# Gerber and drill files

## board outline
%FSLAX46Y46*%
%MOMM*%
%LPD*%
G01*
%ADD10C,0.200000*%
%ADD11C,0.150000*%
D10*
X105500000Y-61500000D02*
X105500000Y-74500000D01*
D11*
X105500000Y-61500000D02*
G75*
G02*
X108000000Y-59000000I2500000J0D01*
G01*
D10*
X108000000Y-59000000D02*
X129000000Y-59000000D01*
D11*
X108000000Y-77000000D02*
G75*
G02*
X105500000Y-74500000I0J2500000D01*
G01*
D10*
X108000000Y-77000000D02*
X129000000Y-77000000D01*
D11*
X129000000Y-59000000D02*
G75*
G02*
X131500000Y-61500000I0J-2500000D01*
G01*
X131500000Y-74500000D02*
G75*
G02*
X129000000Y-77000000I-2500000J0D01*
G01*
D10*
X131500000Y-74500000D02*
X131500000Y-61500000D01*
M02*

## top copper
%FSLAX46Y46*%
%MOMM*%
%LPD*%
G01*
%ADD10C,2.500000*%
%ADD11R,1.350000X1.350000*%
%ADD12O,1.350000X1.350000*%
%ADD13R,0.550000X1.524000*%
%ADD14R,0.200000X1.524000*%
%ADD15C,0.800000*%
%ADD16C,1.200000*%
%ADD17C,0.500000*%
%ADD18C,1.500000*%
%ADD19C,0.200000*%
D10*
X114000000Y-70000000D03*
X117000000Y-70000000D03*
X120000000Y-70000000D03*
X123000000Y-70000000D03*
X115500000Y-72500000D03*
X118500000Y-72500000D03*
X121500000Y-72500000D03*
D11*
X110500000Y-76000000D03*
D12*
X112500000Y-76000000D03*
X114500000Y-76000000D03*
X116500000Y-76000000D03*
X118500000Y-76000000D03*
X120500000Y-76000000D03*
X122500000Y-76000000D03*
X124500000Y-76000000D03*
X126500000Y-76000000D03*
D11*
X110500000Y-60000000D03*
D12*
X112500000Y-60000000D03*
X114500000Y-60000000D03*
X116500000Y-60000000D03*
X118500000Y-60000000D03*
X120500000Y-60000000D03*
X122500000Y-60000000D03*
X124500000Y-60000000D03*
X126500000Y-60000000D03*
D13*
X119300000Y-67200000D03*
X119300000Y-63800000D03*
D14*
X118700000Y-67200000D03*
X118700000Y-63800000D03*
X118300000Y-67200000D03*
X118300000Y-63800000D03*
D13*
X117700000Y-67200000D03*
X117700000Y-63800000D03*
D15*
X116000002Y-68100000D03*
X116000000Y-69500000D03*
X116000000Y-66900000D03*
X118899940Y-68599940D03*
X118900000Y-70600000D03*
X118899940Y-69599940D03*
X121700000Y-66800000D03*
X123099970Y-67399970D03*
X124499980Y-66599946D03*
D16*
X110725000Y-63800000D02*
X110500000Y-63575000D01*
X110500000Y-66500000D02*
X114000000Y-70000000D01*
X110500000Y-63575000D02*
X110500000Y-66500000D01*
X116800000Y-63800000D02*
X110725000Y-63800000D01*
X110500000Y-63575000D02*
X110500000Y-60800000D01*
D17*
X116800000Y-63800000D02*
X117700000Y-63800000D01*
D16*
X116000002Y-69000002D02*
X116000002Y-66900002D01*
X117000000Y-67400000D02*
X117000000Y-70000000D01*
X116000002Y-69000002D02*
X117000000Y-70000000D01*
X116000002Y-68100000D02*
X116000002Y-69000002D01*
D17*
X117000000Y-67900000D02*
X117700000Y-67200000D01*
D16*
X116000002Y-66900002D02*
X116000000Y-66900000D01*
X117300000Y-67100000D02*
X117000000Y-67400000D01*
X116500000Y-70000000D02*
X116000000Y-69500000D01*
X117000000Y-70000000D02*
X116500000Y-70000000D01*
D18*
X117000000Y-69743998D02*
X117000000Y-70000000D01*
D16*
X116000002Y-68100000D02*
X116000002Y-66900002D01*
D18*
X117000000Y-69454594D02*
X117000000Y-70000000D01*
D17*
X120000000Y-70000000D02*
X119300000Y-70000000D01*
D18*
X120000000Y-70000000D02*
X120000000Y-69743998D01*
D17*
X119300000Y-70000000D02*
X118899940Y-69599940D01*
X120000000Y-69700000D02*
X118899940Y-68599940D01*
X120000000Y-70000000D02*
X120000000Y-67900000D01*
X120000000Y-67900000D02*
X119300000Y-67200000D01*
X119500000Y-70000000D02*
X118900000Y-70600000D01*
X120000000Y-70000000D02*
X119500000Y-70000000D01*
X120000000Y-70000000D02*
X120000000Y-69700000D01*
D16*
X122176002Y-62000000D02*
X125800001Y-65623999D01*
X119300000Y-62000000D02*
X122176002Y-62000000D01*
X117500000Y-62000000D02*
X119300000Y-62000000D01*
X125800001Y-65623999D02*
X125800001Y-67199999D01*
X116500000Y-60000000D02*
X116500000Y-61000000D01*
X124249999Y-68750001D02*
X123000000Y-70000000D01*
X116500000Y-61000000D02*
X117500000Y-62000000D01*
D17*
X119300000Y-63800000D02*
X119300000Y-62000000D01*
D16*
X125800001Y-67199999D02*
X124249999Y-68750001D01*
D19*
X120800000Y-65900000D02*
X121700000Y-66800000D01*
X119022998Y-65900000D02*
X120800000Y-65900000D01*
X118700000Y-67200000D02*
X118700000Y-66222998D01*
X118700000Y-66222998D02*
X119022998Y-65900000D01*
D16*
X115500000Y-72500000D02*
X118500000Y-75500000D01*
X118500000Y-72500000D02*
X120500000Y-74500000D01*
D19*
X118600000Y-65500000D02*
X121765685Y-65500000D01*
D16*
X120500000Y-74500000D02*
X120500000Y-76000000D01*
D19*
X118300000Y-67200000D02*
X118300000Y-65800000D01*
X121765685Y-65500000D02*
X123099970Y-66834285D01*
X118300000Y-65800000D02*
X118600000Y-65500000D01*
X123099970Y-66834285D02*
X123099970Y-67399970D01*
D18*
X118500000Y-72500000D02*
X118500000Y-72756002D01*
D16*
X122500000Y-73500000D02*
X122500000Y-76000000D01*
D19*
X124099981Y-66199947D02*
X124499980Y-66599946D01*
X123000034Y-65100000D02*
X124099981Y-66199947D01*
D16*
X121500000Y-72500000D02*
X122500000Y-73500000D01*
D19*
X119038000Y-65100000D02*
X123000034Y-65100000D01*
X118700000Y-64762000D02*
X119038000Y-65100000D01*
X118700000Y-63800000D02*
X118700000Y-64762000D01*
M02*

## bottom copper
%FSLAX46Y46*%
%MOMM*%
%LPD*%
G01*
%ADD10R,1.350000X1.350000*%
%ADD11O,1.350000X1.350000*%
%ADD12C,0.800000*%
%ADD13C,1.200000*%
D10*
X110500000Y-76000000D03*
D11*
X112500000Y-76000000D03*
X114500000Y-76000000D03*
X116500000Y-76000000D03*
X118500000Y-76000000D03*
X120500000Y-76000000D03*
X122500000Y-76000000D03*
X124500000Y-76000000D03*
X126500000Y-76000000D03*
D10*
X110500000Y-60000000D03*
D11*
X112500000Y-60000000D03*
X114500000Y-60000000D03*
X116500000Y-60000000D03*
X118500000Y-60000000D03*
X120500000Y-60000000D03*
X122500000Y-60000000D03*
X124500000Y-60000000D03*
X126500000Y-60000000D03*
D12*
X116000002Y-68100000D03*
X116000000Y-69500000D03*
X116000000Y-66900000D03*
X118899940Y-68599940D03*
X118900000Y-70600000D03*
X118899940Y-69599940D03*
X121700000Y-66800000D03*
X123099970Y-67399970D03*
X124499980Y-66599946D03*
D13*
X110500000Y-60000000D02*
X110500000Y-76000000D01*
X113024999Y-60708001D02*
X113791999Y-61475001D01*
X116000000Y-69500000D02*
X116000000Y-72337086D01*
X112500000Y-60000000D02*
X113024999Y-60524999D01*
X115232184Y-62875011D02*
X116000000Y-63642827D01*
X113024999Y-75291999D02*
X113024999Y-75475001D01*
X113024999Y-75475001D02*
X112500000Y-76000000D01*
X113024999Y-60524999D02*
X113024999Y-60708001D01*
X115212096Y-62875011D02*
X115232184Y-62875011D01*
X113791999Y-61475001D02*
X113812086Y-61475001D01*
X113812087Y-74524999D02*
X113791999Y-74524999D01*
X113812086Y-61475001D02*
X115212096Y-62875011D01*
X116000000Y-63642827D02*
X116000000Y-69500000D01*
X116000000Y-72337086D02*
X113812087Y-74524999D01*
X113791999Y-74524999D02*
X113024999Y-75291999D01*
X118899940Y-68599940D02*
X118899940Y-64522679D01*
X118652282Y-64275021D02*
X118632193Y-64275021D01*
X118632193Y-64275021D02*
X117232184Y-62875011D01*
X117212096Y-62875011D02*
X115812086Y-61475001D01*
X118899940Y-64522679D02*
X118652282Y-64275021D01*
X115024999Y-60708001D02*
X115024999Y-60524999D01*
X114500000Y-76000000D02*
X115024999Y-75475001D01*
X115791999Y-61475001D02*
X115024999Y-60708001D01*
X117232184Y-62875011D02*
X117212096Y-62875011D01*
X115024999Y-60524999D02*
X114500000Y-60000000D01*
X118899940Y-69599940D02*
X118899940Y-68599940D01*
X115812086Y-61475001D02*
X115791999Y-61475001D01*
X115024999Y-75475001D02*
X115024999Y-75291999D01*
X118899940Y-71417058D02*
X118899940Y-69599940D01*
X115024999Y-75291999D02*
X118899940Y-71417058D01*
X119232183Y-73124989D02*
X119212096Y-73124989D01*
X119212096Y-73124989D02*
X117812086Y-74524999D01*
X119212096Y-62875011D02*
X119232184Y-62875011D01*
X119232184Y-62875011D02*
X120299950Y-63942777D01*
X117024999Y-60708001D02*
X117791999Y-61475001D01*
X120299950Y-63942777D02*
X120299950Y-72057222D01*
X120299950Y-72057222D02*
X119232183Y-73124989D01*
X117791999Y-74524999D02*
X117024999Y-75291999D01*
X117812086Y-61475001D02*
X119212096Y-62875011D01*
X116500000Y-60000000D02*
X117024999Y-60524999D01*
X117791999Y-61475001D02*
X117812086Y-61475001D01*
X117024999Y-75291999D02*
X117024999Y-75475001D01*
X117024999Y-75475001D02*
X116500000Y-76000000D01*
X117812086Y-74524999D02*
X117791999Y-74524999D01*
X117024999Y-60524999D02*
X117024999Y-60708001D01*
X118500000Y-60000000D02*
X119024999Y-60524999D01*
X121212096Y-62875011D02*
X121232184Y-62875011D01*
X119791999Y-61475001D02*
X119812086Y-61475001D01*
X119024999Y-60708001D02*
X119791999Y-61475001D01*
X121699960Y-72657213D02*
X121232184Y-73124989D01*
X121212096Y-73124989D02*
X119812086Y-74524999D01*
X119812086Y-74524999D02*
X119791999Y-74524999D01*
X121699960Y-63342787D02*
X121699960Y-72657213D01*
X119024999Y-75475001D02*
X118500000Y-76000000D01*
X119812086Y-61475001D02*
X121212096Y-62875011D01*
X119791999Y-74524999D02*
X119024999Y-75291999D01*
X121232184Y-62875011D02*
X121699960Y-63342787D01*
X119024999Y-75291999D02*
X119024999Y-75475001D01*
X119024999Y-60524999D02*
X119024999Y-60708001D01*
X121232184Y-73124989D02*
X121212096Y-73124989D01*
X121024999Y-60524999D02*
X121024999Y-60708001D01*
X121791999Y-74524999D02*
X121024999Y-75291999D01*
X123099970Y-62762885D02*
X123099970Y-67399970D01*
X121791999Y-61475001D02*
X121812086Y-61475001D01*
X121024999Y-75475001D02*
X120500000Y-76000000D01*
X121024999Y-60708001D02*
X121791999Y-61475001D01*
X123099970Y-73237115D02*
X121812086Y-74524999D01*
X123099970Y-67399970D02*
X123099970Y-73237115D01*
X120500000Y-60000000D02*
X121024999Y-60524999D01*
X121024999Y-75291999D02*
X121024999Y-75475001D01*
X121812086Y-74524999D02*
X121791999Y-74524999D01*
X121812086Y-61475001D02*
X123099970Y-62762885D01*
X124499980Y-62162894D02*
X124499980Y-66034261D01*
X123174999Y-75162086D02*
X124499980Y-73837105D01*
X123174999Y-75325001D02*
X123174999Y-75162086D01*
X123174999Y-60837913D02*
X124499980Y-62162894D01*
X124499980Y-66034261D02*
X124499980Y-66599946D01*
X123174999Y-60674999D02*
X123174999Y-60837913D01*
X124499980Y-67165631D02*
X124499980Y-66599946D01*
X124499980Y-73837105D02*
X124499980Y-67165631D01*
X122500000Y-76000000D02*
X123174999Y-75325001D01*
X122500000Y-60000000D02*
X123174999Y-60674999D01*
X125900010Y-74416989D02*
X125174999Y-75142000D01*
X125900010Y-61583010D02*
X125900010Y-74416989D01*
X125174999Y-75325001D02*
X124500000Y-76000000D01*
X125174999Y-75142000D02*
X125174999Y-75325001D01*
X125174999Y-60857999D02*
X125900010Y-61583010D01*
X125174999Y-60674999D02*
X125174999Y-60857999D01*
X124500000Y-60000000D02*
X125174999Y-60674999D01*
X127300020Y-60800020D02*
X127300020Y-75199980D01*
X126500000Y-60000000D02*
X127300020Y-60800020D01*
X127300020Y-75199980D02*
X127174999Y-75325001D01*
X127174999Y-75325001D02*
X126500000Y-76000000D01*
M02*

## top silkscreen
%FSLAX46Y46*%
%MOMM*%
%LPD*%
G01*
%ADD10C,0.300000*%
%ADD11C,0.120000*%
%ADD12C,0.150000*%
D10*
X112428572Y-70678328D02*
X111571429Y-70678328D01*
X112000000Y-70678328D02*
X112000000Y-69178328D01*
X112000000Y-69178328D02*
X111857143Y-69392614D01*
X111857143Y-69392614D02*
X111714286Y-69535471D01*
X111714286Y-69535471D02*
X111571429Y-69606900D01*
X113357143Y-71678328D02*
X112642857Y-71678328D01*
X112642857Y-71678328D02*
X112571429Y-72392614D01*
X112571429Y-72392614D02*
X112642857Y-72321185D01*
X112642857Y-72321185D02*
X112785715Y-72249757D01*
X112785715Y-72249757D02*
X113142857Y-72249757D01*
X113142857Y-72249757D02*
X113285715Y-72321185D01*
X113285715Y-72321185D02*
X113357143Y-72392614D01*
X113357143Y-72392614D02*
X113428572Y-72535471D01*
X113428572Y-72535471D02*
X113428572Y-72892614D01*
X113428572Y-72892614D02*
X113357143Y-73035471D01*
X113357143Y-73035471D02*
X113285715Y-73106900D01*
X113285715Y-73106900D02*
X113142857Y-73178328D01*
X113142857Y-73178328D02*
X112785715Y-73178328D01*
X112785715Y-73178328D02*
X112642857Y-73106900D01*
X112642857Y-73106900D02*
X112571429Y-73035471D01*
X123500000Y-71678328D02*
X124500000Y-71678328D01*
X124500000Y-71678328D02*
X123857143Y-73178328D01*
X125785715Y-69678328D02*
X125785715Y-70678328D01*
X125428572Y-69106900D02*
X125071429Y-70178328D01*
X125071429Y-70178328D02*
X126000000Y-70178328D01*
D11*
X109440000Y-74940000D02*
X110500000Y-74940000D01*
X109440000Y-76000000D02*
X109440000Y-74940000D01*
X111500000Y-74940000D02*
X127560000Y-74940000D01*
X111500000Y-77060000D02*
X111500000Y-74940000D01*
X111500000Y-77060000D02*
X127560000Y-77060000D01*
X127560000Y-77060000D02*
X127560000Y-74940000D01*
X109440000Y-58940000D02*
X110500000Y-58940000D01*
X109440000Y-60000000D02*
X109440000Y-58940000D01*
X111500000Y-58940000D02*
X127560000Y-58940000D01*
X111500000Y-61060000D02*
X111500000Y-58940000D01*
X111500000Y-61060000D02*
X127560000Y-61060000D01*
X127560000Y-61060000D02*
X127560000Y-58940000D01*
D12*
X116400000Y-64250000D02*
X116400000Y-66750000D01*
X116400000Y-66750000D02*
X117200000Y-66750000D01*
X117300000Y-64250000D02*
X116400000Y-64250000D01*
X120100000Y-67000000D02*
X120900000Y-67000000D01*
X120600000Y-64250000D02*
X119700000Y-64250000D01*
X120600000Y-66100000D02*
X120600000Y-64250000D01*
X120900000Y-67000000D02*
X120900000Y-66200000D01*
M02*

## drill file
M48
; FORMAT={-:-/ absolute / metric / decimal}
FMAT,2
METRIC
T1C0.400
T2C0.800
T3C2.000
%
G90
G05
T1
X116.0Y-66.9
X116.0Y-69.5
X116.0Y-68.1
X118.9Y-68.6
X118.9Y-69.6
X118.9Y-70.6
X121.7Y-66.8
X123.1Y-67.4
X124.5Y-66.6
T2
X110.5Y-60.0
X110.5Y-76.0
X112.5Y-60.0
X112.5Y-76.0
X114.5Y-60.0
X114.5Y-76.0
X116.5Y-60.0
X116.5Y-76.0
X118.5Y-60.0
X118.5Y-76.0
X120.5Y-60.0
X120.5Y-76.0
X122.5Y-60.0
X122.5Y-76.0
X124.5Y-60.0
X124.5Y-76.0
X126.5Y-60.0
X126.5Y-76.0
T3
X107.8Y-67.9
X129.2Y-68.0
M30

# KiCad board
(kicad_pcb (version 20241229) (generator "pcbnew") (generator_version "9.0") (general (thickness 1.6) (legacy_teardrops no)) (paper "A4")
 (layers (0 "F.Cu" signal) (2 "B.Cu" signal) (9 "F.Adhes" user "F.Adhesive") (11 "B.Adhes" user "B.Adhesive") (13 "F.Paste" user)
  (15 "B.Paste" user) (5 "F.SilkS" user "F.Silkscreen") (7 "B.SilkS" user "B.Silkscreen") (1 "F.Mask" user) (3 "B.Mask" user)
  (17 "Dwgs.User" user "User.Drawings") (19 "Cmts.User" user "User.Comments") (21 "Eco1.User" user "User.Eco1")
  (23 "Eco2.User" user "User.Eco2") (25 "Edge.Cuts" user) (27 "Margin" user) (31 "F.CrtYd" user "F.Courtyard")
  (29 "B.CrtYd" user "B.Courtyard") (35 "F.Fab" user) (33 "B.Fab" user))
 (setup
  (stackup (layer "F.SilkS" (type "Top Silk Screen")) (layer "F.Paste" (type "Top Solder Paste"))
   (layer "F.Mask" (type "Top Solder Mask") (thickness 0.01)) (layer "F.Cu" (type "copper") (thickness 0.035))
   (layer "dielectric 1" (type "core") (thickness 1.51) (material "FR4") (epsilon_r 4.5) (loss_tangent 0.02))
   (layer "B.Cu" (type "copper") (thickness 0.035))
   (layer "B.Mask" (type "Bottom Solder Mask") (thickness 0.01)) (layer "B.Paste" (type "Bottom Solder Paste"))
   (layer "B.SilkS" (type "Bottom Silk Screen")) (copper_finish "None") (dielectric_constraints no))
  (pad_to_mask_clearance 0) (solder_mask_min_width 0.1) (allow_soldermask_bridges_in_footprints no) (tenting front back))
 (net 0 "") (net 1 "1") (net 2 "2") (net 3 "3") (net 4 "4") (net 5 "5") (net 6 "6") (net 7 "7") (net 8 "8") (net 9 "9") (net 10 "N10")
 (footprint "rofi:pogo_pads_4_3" (layer "F.Cu") (at 118.5 70)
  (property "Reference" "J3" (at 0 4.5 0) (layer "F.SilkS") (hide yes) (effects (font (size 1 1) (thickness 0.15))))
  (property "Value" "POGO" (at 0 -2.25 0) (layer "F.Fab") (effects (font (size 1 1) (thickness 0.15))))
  (pad "1" smd circle (at -4.5 0) (size 2.5 2.5) (layers "F.Cu" "F.Mask" "F.Paste") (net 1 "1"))
  (pad "2" smd circle (at -1.5 0) (size 2.5 2.5) (layers "F.Cu" "F.Mask" "F.Paste") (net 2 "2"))
  (pad "3" smd circle (at 1.5 0) (size 2.5 2.5) (layers "F.Cu" "F.Mask" "F.Paste") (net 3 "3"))
  (pad "4" smd circle (at 4.5 0) (size 2.5 2.5) (layers "F.Cu" "F.Mask" "F.Paste") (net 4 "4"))
  (pad "5" smd circle (at -3 2.5) (size 2.5 2.5) (layers "F.Cu" "F.Mask" "F.Paste") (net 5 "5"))
  (pad "6" smd circle (at 0 2.5) (size 2.5 2.5) (layers "F.Cu" "F.Mask" "F.Paste") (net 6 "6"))
  (pad "7" smd circle (at 3 2.5) (size 2.5 2.5) (layers "F.Cu" "F.Mask" "F.Paste") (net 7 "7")))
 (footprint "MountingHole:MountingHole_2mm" (layer "F.Cu") (at 129.2 68)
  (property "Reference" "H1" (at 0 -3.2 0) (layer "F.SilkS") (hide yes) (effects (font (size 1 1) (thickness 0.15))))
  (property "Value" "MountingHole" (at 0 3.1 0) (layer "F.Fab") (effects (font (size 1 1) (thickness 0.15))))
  (pad "" np_thru_hole circle (at 0 0) (size 2 2) (drill 2) (layers "*.Cu" "*.Mask")))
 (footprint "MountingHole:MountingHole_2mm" (layer "F.Cu") (at 107.8 67.9)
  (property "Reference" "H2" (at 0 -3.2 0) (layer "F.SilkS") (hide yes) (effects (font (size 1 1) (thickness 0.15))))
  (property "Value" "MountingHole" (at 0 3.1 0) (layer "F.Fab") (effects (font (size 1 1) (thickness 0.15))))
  (pad "" np_thru_hole circle (at 0 0) (size 2 2) (drill 2) (layers "*.Cu" "*.Mask")))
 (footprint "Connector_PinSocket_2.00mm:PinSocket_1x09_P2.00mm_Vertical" (layer "F.Cu") (at 110.5 76 90)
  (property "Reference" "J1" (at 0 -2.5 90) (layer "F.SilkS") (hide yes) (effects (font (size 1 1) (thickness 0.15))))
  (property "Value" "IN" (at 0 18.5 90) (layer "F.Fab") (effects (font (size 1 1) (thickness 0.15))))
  (fp_line (start 1.06 -1.06) (end 1.06 0) (stroke (width 0.12) (type solid)) (layer "F.SilkS"))
  (fp_line (start 0 -1.06) (end 1.06 -1.06) (stroke (width 0.12) (type solid)) (layer "F.SilkS"))
  (fp_line (start 1.06 1) (end 1.06 17.06) (stroke (width 0.12) (type solid)) (layer "F.SilkS"))
  (fp_line (start -1.06 1) (end 1.06 1) (stroke (width 0.12) (type solid)) (layer "F.SilkS"))
  (fp_line (start -1.06 1) (end -1.06 17.06) (stroke (width 0.12) (type solid)) (layer "F.SilkS"))
  (fp_line (start -1.06 17.06) (end 1.06 17.06) (stroke (width 0.12) (type solid)) (layer "F.SilkS"))
  (pad "1" thru_hole rect (at 0 0 90) (size 1.35 1.35) (drill 0.8) (layers "*.Cu" "*.Mask") (remove_unused_layers no) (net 1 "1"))
  (pad "2" thru_hole oval (at 0 2 90) (size 1.35 1.35) (drill 0.8) (layers "*.Cu" "*.Mask") (remove_unused_layers no) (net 2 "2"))
  (pad "3" thru_hole oval (at 0 4 90) (size 1.35 1.35) (drill 0.8) (layers "*.Cu" "*.Mask") (remove_unused_layers no) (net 3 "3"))
  (pad "4" thru_hole oval (at 0 6 90) (size 1.35 1.35) (drill 0.8) (layers "*.Cu" "*.Mask") (remove_unused_layers no) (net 4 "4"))
  (pad "5" thru_hole oval (at 0 8 90) (size 1.35 1.35) (drill 0.8) (layers "*.Cu" "*.Mask") (remove_unused_layers no) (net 5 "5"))
  (pad "6" thru_hole oval (at 0 10 90) (size 1.35 1.35) (drill 0.8) (layers "*.Cu" "*.Mask") (remove_unused_layers no) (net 6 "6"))
  (pad "7" thru_hole oval (at 0 12 90) (size 1.35 1.35) (drill 0.8) (layers "*.Cu" "*.Mask") (remove_unused_layers no) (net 7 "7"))
  (pad "8" thru_hole oval (at 0 14 90) (size 1.35 1.35) (drill 0.8) (layers "*.Cu" "*.Mask") (remove_unused_layers no) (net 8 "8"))
  (pad "9" thru_hole oval (at 0 16 90) (size 1.35 1.35) (drill 0.8) (layers "*.Cu" "*.Mask") (remove_unused_layers no) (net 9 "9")))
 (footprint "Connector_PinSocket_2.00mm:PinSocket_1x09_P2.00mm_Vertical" (layer "F.Cu") (at 110.5 60 90)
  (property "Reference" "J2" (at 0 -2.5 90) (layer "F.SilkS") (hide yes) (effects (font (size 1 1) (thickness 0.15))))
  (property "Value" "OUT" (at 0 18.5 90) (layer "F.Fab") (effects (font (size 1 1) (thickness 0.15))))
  (fp_line (start 1.06 -1.06) (end 1.06 0) (stroke (width 0.12) (type solid)) (layer "F.SilkS"))
  (fp_line (start 0 -1.06) (end 1.06 -1.06) (stroke (width 0.12) (type solid)) (layer "F.SilkS"))
  (fp_line (start 1.06 1) (end 1.06 17.06) (stroke (width 0.12) (type solid)) (layer "F.SilkS"))
  (fp_line (start -1.06 1) (end 1.06 1) (stroke (width 0.12) (type solid)) (layer "F.SilkS"))
  (fp_line (start -1.06 1) (end -1.06 17.06) (stroke (width 0.12) (type solid)) (layer "F.SilkS"))
  (fp_line (start -1.06 17.06) (end 1.06 17.06) (stroke (width 0.12) (type solid)) (layer "F.SilkS"))
  (pad "1" thru_hole rect (at 0 0 90) (size 1.35 1.35) (drill 0.8) (layers "*.Cu" "*.Mask") (remove_unused_layers no) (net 1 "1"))
  (pad "2" thru_hole oval (at 0 2 90) (size 1.35 1.35) (drill 0.8) (layers "*.Cu" "*.Mask") (remove_unused_layers no) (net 2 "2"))
  (pad "3" thru_hole oval (at 0 4 90) (size 1.35 1.35) (drill 0.8) (layers "*.Cu" "*.Mask") (remove_unused_layers no) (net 3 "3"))
  (pad "4" thru_hole oval (at 0 6 90) (size 1.35 1.35) (drill 0.8) (layers "*.Cu" "*.Mask") (remove_unused_layers no) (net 4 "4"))
  (pad "5" thru_hole oval (at 0 8 90) (size 1.35 1.35) (drill 0.8) (layers "*.Cu" "*.Mask") (remove_unused_layers no) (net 5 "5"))
  (pad "6" thru_hole oval (at 0 10 90) (size 1.35 1.35) (drill 0.8) (layers "*.Cu" "*.Mask") (remove_unused_layers no) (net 6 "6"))
  (pad "7" thru_hole oval (at 0 12 90) (size 1.35 1.35) (drill 0.8) (layers "*.Cu" "*.Mask") (remove_unused_layers no) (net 7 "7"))
  (pad "8" thru_hole oval (at 0 14 90) (size 1.35 1.35) (drill 0.8) (layers "*.Cu" "*.Mask") (remove_unused_layers no) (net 8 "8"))
  (pad "9" thru_hole oval (at 0 16 90) (size 1.35 1.35) (drill 0.8) (layers "*.Cu" "*.Mask") (remove_unused_layers no) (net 9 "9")))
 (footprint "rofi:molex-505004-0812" (layer "F.Cu") (at 118.5 65.5 180)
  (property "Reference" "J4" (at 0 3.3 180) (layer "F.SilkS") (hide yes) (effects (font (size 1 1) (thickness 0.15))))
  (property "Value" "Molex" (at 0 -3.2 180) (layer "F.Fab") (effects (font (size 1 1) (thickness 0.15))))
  (fp_line (start 2.1 1.25) (end 2.1 -1.25) (stroke (width 0.15) (type solid)) (layer "F.SilkS"))
  (fp_line (start 2.1 -1.25) (end 1.3 -1.25) (stroke (width 0.15) (type solid)) (layer "F.SilkS"))
  (fp_line (start 1.2 1.25) (end 2.1 1.25) (stroke (width 0.15) (type solid)) (layer "F.SilkS"))
  (fp_line (start -1.6 -1.5) (end -2.4 -1.5) (stroke (width 0.15) (type solid)) (layer "F.SilkS"))
  (fp_line (start -2.1 1.25) (end -1.2 1.25) (stroke (width 0.15) (type solid)) (layer "F.SilkS"))
  (fp_line (start -2.1 -0.6) (end -2.1 1.25) (stroke (width 0.15) (type solid)) (layer "F.SilkS"))
  (fp_line (start -2.4 -1.5) (end -2.4 -0.7) (stroke (width 0.15) (type solid)) (layer "F.SilkS"))
  (pad "1" smd rect (at -0.8 -1.7 180) (size 0.55 1.524) (layers "F.Cu" "F.Mask" "F.Paste") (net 3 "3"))
  (pad "2" smd rect (at -0.8 1.7 180) (size 0.55 1.524) (layers "F.Cu" "F.Mask" "F.Paste") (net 4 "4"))
  (pad "3" smd rect (at -0.2 -1.7 180) (size 0.2 1.524) (layers "F.Cu" "F.Mask" "F.Paste") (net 5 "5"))
  (pad "4" smd rect (at -0.2 1.7 180) (size 0.2 1.524) (layers "F.Cu" "F.Mask" "F.Paste") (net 7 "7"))
  (pad "5" smd rect (at 0.2 -1.7 180) (size 0.2 1.524) (layers "F.Cu" "F.Mask" "F.Paste") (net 6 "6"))
  (pad "6" smd rect (at 0.2 1.7 180) (size 0.2 1.524) (layers "F.Cu" "F.Mask" "F.Paste") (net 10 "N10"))
  (pad "7" smd rect (at 0.8 -1.7 180) (size 0.55 1.524) (layers "F.Cu" "F.Mask" "F.Paste") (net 2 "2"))
  (pad "8" smd rect (at 0.8 1.7 180) (size 0.55 1.524) (layers "F.Cu" "F.Mask" "F.Paste") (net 1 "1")))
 (gr_line (start 105.5 61.5) (end 105.5 74.5) (stroke (width 0.2) (type solid)) (layer "Edge.Cuts"))
 (gr_arc (start 105.5 61.5) (mid 106.232233 59.732233) (end 108 59) (stroke (width 0.15) (type solid)) (layer "Edge.Cuts"))
 (gr_line (start 108 59) (end 129 59) (stroke (width 0.2) (type solid)) (layer "Edge.Cuts"))
 (gr_arc (start 108 77) (mid 106.232233 76.267767) (end 105.5 74.5) (stroke (width 0.15) (type solid)) (layer "Edge.Cuts"))
 (gr_line (start 108 77) (end 129 77) (stroke (width 0.2) (type solid)) (layer "Edge.Cuts"))
 (gr_arc (start 129 59) (mid 130.767767 59.732233) (end 131.5 61.5) (stroke (width 0.15) (type solid)) (layer "Edge.Cuts"))
 (gr_arc (start 131.5 74.5) (mid 130.767767 76.267767) (end 129 77) (stroke (width 0.15) (type solid)) (layer "Edge.Cuts"))
 (gr_line (start 131.5 74.5) (end 131.5 61.5) (stroke (width 0.2) (type solid)) (layer "Edge.Cuts"))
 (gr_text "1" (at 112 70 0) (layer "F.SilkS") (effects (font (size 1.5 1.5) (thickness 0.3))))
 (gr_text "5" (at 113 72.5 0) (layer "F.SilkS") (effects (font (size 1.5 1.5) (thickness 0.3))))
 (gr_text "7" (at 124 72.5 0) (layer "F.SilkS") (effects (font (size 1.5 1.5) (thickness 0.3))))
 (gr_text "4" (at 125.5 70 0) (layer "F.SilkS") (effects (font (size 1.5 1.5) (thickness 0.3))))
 (segment (start 110.725 63.8) (end 110.5 63.575) (width 1.2) (layer "F.Cu") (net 1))
 (segment (start 110.5 66.5) (end 114 70) (width 1.2) (layer "F.Cu") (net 1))
 (segment (start 110.5 63.575) (end 110.5 66.5) (width 1.2) (layer "F.Cu") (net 1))
 (segment (start 116.8 63.8) (end 110.725 63.8) (width 1.2) (layer "F.Cu") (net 1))
 (segment (start 110.5 63.575) (end 110.5 60.8) (width 1.2) (layer "F.Cu") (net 1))
 (segment (start 116.8 63.8) (end 117.7 63.8) (width 0.5) (layer "F.Cu") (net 1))
 (segment (start 110.5 60) (end 110.5 76) (width 1.2) (layer "B.Cu") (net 1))
 (segment (start 116.000002 69.000002) (end 116.000002 66.900002) (width 1.2) (layer "F.Cu") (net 2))
 (segment (start 117 67.4) (end 117 70) (width 1.2) (layer "F.Cu") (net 2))
 (segment (start 116.000002 69.000002) (end 117 70) (width 1.2) (layer "F.Cu") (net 2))
 (segment (start 116.000002 68.1) (end 116.000002 69.000002) (width 1.2) (layer "F.Cu") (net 2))
 (segment (start 117 67.9) (end 117.7 67.2) (width 0.5) (layer "F.Cu") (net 2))
 (segment (start 116.000002 66.900002) (end 116 66.9) (width 1.2) (layer "F.Cu") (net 2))
 (segment (start 117.3 67.1) (end 117 67.4) (width 1.2) (layer "F.Cu") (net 2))
 (segment (start 116.5 70) (end 116 69.5) (width 1.2) (layer "F.Cu") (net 2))
 (segment (start 117 70) (end 116.5 70) (width 1.2) (layer "F.Cu") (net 2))
 (segment (start 117 69.743998) (end 117 70) (width 1.5) (layer "F.Cu") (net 2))
 (segment (start 116.000002 68.1) (end 116.000002 66.900002) (width 1.2) (layer "F.Cu") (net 2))
 (segment (start 117 69.454594) (end 117 70) (width 1.5) (layer "F.Cu") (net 2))
 (via (at 116.000002 68.1) (size 0.8) (drill 0.4) (layers "F.Cu" "B.Cu") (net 2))
 (via (at 116 69.5) (size 0.8) (drill 0.4) (layers "F.Cu" "B.Cu") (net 2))
 (via (at 116 66.9) (size 0.8) (drill 0.4) (layers "F.Cu" "B.Cu") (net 2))
 (segment (start 113.024999 60.708001) (end 113.791999 61.475001) (width 1.2) (layer "B.Cu") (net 2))
 (segment (start 116 69.5) (end 116 72.337086) (width 1.2) (layer "B.Cu") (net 2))
 (segment (start 112.5 60) (end 113.024999 60.524999) (width 1.2) (layer "B.Cu") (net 2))
 (segment (start 115.232184 62.875011) (end 116 63.642827) (width 1.2) (layer "B.Cu") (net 2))
 (segment (start 113.024999 75.291999) (end 113.024999 75.475001) (width 1.2) (layer "B.Cu") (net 2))
 (segment (start 113.024999 75.475001) (end 112.5 76) (width 1.2) (layer "B.Cu") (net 2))
 (segment (start 113.024999 60.524999) (end 113.024999 60.708001) (width 1.2) (layer "B.Cu") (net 2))
 (segment (start 115.212096 62.875011) (end 115.232184 62.875011) (width 1.2) (layer "B.Cu") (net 2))
 (segment (start 113.791999 61.475001) (end 113.812086 61.475001) (width 1.2) (layer "B.Cu") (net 2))
 (segment (start 113.812087 74.524999) (end 113.791999 74.524999) (width 1.2) (layer "B.Cu") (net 2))
 (segment (start 113.812086 61.475001) (end 115.212096 62.875011) (width 1.2) (layer "B.Cu") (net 2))
 (segment (start 116 63.642827) (end 116 69.5) (width 1.2) (layer "B.Cu") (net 2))
 (segment (start 116 72.337086) (end 113.812087 74.524999) (width 1.2) (layer "B.Cu") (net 2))
 (segment (start 113.791999 74.524999) (end 113.024999 75.291999) (width 1.2) (layer "B.Cu") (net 2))
 (segment (start 120 70) (end 119.3 70) (width 0.5) (layer "F.Cu") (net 3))
 (segment (start 120 70) (end 120 69.743998) (width 1.5) (layer "F.Cu") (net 3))
 (segment (start 119.3 70) (end 118.89994 69.59994) (width 0.5) (layer "F.Cu") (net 3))
 (segment (start 120 69.7) (end 118.89994 68.59994) (width 0.5) (layer "F.Cu") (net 3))
 (segment (start 120 70) (end 120 67.9) (width 0.5) (layer "F.Cu") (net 3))
 (segment (start 120 67.9) (end 119.3 67.2) (width 0.5) (layer "F.Cu") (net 3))
 (segment (start 119.5 70) (end 118.9 70.6) (width 0.5) (layer "F.Cu") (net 3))
 (segment (start 120 70) (end 119.5 70) (width 0.5) (layer "F.Cu") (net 3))
 (segment (start 120 70) (end 120 69.7) (width 0.5) (layer "F.Cu") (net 3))
 (via (at 118.89994 68.59994) (size 0.8) (drill 0.4) (layers "F.Cu" "B.Cu") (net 3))
 (via (at 118.9 70.6) (size 0.8) (drill 0.4) (layers "F.Cu" "B.Cu") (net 3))
 (via (at 118.89994 69.59994) (size 0.8) (drill 0.4) (layers "F.Cu" "B.Cu") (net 3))
 (segment (start 118.89994 68.59994) (end 118.89994 64.522679) (width 1.2) (layer "B.Cu") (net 3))
 (segment (start 118.652282 64.275021) (end 118.632193 64.275021) (width 1.2) (layer "B.Cu") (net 3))
 (segment (start 118.632193 64.275021) (end 117.232184 62.875011) (width 1.2) (layer "B.Cu") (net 3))
 (segment (start 117.212096 62.875011) (end 115.812086 61.475001) (width 1.2) (layer "B.Cu") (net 3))
 (segment (start 118.89994 64.522679) (end 118.652282 64.275021) (width 1.2) (layer "B.Cu") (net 3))
 (segment (start 115.024999 60.708001) (end 115.024999 60.524999) (width 1.2) (layer "B.Cu") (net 3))
 (segment (start 114.5 76) (end 115.024999 75.475001) (width 1.2) (layer "B.Cu") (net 3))
 (segment (start 115.791999 61.475001) (end 115.024999 60.708001) (width 1.2) (layer "B.Cu") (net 3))
 (segment (start 117.232184 62.875011) (end 117.212096 62.875011) (width 1.2) (layer "B.Cu") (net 3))
 (segment (start 115.024999 60.524999) (end 114.5 60) (width 1.2) (layer "B.Cu") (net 3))
 (segment (start 118.89994 69.59994) (end 118.89994 68.59994) (width 1.2) (layer "B.Cu") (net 3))
 (segment (start 115.812086 61.475001) (end 115.791999 61.475001) (width 1.2) (layer "B.Cu") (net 3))
 (segment (start 115.024999 75.475001) (end 115.024999 75.291999) (width 1.2) (layer "B.Cu") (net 3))
 (segment (start 118.89994 71.417058) (end 118.89994 69.59994) (width 1.2) (layer "B.Cu") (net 3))
 (segment (start 115.024999 75.291999) (end 118.89994 71.417058) (width 1.2) (layer "B.Cu") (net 3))
 (segment (start 122.176002 62) (end 125.800001 65.623999) (width 1.2) (layer "F.Cu") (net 4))
 (segment (start 119.3 62) (end 122.176002 62) (width 1.2) (layer "F.Cu") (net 4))
 (segment (start 117.5 62) (end 119.3 62) (width 1.2) (layer "F.Cu") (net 4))
 (segment (start 125.800001 65.623999) (end 125.800001 67.199999) (width 1.2) (layer "F.Cu") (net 4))
 (segment (start 116.5 60) (end 116.5 61) (width 1.2) (layer "F.Cu") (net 4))
 (segment (start 124.249999 68.750001) (end 123 70) (width 1.2) (layer "F.Cu") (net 4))
 (segment (start 116.5 61) (end 117.5 62) (width 1.2) (layer "F.Cu") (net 4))
 (segment (start 119.3 63.8) (end 119.3 62) (width 0.5) (layer "F.Cu") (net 4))
 (segment (start 125.800001 67.199999) (end 124.249999 68.750001) (width 1.2) (layer "F.Cu") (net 4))
 (segment (start 119.232183 73.124989) (end 119.212096 73.124989) (width 1.2) (layer "B.Cu") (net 4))
 (segment (start 119.212096 73.124989) (end 117.812086 74.524999) (width 1.2) (layer "B.Cu") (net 4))
 (segment (start 119.212096 62.875011) (end 119.232184 62.875011) (width 1.2) (layer "B.Cu") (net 4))
 (segment (start 119.232184 62.875011) (end 120.29995 63.942777) (width 1.2) (layer "B.Cu") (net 4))
 (segment (start 117.024999 60.708001) (end 117.791999 61.475001) (width 1.2) (layer "B.Cu") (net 4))
 (segment (start 120.29995 63.942777) (end 120.29995 72.057222) (width 1.2) (layer "B.Cu") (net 4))
 (segment (start 120.29995 72.057222) (end 119.232183 73.124989) (width 1.2) (layer "B.Cu") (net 4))
 (segment (start 117.791999 74.524999) (end 117.024999 75.291999) (width 1.2) (layer "B.Cu") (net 4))
 (segment (start 117.812086 61.475001) (end 119.212096 62.875011) (width 1.2) (layer "B.Cu") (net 4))
 (segment (start 116.5 60) (end 117.024999 60.524999) (width 1.2) (layer "B.Cu") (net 4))
 (segment (start 117.791999 61.475001) (end 117.812086 61.475001) (width 1.2) (layer "B.Cu") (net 4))
 (segment (start 117.024999 75.291999) (end 117.024999 75.475001) (width 1.2) (layer "B.Cu") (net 4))
 (segment (start 117.024999 75.475001) (end 116.5 76) (width 1.2) (layer "B.Cu") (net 4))
 (segment (start 117.812086 74.524999) (end 117.791999 74.524999) (width 1.2) (layer "B.Cu") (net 4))
 (segment (start 117.024999 60.524999) (end 117.024999 60.708001) (width 1.2) (layer "B.Cu") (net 4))
 (segment (start 120.8 65.9) (end 121.7 66.8) (width 0.2) (layer "F.Cu") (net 5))
 (segment (start 119.022998 65.9) (end 120.8 65.9) (width 0.2) (layer "F.Cu") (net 5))
 (segment (start 118.7 67.2) (end 118.7 66.222998) (width 0.2) (layer "F.Cu") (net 5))
 (segment (start 118.7 66.222998) (end 119.022998 65.9) (width 0.2) (layer "F.Cu") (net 5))
 (segment (start 115.5 72.5) (end 118.5 75.5) (width 1.2) (layer "F.Cu") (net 5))
 (via (at 121.7 66.8) (size 0.8) (drill 0.4) (layers "F.Cu" "B.Cu") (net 5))
 (segment (start 118.5 60) (end 119.024999 60.524999) (width 1.2) (layer "B.Cu") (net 5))
 (segment (start 121.212096 62.875011) (end 121.232184 62.875011) (width 1.2) (layer "B.Cu") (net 5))
 (segment (start 119.791999 61.475001) (end 119.812086 61.475001) (width 1.2) (layer "B.Cu") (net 5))
 (segment (start 119.024999 60.708001) (end 119.791999 61.475001) (width 1.2) (layer "B.Cu") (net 5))
 (segment (start 121.69996 72.657213) (end 121.232184 73.124989) (width 1.2) (layer "B.Cu") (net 5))
 (segment (start 121.212096 73.124989) (end 119.812086 74.524999) (width 1.2) (layer "B.Cu") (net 5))
 (segment (start 119.812086 74.524999) (end 119.791999 74.524999) (width 1.2) (layer "B.Cu") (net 5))
 (segment (start 121.69996 63.342787) (end 121.69996 72.657213) (width 1.2) (layer "B.Cu") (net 5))
 (segment (start 119.024999 75.475001) (end 118.5 76) (width 1.2) (layer "B.Cu") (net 5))
 (segment (start 119.812086 61.475001) (end 121.212096 62.875011) (width 1.2) (layer "B.Cu") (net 5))
 (segment (start 119.791999 74.524999) (end 119.024999 75.291999) (width 1.2) (layer "B.Cu") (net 5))
 (segment (start 121.232184 62.875011) (end 121.69996 63.342787) (width 1.2) (layer "B.Cu") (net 5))
 (segment (start 119.024999 75.291999) (end 119.024999 75.475001) (width 1.2) (layer "B.Cu") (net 5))
 (segment (start 119.024999 60.524999) (end 119.024999 60.708001) (width 1.2) (layer "B.Cu") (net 5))
 (segment (start 121.232184 73.124989) (end 121.212096 73.124989) (width 1.2) (layer "B.Cu") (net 5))
 (segment (start 118.5 72.5) (end 120.5 74.5) (width 1.2) (layer "F.Cu") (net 6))
 (segment (start 118.6 65.5) (end 121.765685 65.5) (width 0.2) (layer "F.Cu") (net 6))
 (segment (start 120.5 74.5) (end 120.5 76) (width 1.2) (layer "F.Cu") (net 6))
 (segment (start 118.3 67.2) (end 118.3 65.8) (width 0.2) (layer "F.Cu") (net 6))
 (segment (start 121.765685 65.5) (end 123.09997 66.834285) (width 0.2) (layer "F.Cu") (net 6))
 (segment (start 118.3 65.8) (end 118.6 65.5) (width 0.2) (layer "F.Cu") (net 6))
 (segment (start 123.09997 66.834285) (end 123.09997 67.39997) (width 0.2) (layer "F.Cu") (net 6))
 (segment (start 118.5 72.5) (end 118.5 72.756002) (width 1.5) (layer "F.Cu") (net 6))
 (via (at 123.09997 67.39997) (size 0.8) (drill 0.4) (layers "F.Cu" "B.Cu") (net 6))
 (segment (start 121.024999 60.524999) (end 121.024999 60.708001) (width 1.2) (layer "B.Cu") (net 6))
 (segment (start 121.791999 74.524999) (end 121.024999 75.291999) (width 1.2) (layer "B.Cu") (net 6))
 (segment (start 123.09997 62.762885) (end 123.09997 67.39997) (width 1.2) (layer "B.Cu") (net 6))
 (segment (start 121.791999 61.475001) (end 121.812086 61.475001) (width 1.2) (layer "B.Cu") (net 6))
 (segment (start 121.024999 75.475001) (end 120.5 76) (width 1.2) (layer "B.Cu") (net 6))
 (segment (start 121.024999 60.708001) (end 121.791999 61.475001) (width 1.2) (layer "B.Cu") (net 6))
 (segment (start 123.09997 73.237115) (end 121.812086 74.524999) (width 1.2) (layer "B.Cu") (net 6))
 (segment (start 123.09997 67.39997) (end 123.09997 73.237115) (width 1.2) (layer "B.Cu") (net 6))
 (segment (start 120.5 60) (end 121.024999 60.524999) (width 1.2) (layer "B.Cu") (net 6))
 (segment (start 121.024999 75.291999) (end 121.024999 75.475001) (width 1.2) (layer "B.Cu") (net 6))
 (segment (start 121.812086 74.524999) (end 121.791999 74.524999) (width 1.2) (layer "B.Cu") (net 6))
 (segment (start 121.812086 61.475001) (end 123.09997 62.762885) (width 1.2) (layer "B.Cu") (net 6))
 (segment (start 122.5 73.5) (end 122.5 76) (width 1.2) (layer "F.Cu") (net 7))
 (segment (start 124.099981 66.199947) (end 124.49998 66.599946) (width 0.2) (layer "F.Cu") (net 7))
 (segment (start 123.000034 65.1) (end 124.099981 66.199947) (width 0.2) (layer "F.Cu") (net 7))
 (segment (start 121.5 72.5) (end 122.5 73.5) (width 1.2) (layer "F.Cu") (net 7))
 (segment (start 119.038 65.1) (end 123.000034 65.1) (width 0.2) (layer "F.Cu") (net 7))
 (segment (start 118.7 64.762) (end 119.038 65.1) (width 0.2) (layer "F.Cu") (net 7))
 (segment (start 118.7 63.8) (end 118.7 64.762) (width 0.2) (layer "F.Cu") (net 7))
 (via (at 124.49998 66.599946) (size 0.8) (drill 0.4) (layers "F.Cu" "B.Cu") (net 7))
 (segment (start 124.49998 62.162894) (end 124.49998 66.034261) (width 1.2) (layer "B.Cu") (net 7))
 (segment (start 123.174999 75.162086) (end 124.49998 73.837105) (width 1.2) (layer "B.Cu") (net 7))
 (segment (start 123.174999 75.325001) (end 123.174999 75.162086) (width 1.2) (layer "B.Cu") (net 7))
 (segment (start 123.174999 60.837913) (end 124.49998 62.162894) (width 1.2) (layer "B.Cu") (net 7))
 (segment (start 124.49998 66.034261) (end 124.49998 66.599946) (width 1.2) (layer "B.Cu") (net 7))
 (segment (start 123.174999 60.674999) (end 123.174999 60.837913) (width 1.2) (layer "B.Cu") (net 7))
 (segment (start 124.49998 67.165631) (end 124.49998 66.599946) (width 1.2) (layer "B.Cu") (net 7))
 (segment (start 124.49998 73.837105) (end 124.49998 67.165631) (width 1.2) (layer "B.Cu") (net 7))
 (segment (start 122.5 76) (end 123.174999 75.325001) (width 1.2) (layer "B.Cu") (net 7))
 (segment (start 122.5 60) (end 123.174999 60.674999) (width 1.2) (layer "B.Cu") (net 7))
 (segment (start 125.90001 74.416989) (end 125.174999 75.142) (width 1.2) (layer "B.Cu") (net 8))
 (segment (start 125.90001 61.58301) (end 125.90001 74.416989) (width 1.2) (layer "B.Cu") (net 8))
 (segment (start 125.174999 75.325001) (end 124.5 76) (width 1.2) (layer "B.Cu") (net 8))
 (segment (start 125.174999 75.142) (end 125.174999 75.325001) (width 1.2) (layer "B.Cu") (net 8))
 (segment (start 125.174999 60.857999) (end 125.90001 61.58301) (width 1.2) (layer "B.Cu") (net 8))
 (segment (start 125.174999 60.674999) (end 125.174999 60.857999) (width 1.2) (layer "B.Cu") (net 8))
 (segment (start 124.5 60) (end 125.174999 60.674999) (width 1.2) (layer "B.Cu") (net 8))
 (segment (start 127.30002 60.80002) (end 127.30002 75.19998) (width 1.2) (layer "B.Cu") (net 9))
 (segment (start 126.5 60) (end 127.30002 60.80002) (width 1.2) (layer "B.Cu") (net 9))
 (segment (start 127.30002 75.19998) (end 127.174999 75.325001) (width 1.2) (layer "B.Cu") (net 9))
 (segment (start 127.174999 75.325001) (end 126.5 76) (width 1.2) (layer "B.Cu") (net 9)))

